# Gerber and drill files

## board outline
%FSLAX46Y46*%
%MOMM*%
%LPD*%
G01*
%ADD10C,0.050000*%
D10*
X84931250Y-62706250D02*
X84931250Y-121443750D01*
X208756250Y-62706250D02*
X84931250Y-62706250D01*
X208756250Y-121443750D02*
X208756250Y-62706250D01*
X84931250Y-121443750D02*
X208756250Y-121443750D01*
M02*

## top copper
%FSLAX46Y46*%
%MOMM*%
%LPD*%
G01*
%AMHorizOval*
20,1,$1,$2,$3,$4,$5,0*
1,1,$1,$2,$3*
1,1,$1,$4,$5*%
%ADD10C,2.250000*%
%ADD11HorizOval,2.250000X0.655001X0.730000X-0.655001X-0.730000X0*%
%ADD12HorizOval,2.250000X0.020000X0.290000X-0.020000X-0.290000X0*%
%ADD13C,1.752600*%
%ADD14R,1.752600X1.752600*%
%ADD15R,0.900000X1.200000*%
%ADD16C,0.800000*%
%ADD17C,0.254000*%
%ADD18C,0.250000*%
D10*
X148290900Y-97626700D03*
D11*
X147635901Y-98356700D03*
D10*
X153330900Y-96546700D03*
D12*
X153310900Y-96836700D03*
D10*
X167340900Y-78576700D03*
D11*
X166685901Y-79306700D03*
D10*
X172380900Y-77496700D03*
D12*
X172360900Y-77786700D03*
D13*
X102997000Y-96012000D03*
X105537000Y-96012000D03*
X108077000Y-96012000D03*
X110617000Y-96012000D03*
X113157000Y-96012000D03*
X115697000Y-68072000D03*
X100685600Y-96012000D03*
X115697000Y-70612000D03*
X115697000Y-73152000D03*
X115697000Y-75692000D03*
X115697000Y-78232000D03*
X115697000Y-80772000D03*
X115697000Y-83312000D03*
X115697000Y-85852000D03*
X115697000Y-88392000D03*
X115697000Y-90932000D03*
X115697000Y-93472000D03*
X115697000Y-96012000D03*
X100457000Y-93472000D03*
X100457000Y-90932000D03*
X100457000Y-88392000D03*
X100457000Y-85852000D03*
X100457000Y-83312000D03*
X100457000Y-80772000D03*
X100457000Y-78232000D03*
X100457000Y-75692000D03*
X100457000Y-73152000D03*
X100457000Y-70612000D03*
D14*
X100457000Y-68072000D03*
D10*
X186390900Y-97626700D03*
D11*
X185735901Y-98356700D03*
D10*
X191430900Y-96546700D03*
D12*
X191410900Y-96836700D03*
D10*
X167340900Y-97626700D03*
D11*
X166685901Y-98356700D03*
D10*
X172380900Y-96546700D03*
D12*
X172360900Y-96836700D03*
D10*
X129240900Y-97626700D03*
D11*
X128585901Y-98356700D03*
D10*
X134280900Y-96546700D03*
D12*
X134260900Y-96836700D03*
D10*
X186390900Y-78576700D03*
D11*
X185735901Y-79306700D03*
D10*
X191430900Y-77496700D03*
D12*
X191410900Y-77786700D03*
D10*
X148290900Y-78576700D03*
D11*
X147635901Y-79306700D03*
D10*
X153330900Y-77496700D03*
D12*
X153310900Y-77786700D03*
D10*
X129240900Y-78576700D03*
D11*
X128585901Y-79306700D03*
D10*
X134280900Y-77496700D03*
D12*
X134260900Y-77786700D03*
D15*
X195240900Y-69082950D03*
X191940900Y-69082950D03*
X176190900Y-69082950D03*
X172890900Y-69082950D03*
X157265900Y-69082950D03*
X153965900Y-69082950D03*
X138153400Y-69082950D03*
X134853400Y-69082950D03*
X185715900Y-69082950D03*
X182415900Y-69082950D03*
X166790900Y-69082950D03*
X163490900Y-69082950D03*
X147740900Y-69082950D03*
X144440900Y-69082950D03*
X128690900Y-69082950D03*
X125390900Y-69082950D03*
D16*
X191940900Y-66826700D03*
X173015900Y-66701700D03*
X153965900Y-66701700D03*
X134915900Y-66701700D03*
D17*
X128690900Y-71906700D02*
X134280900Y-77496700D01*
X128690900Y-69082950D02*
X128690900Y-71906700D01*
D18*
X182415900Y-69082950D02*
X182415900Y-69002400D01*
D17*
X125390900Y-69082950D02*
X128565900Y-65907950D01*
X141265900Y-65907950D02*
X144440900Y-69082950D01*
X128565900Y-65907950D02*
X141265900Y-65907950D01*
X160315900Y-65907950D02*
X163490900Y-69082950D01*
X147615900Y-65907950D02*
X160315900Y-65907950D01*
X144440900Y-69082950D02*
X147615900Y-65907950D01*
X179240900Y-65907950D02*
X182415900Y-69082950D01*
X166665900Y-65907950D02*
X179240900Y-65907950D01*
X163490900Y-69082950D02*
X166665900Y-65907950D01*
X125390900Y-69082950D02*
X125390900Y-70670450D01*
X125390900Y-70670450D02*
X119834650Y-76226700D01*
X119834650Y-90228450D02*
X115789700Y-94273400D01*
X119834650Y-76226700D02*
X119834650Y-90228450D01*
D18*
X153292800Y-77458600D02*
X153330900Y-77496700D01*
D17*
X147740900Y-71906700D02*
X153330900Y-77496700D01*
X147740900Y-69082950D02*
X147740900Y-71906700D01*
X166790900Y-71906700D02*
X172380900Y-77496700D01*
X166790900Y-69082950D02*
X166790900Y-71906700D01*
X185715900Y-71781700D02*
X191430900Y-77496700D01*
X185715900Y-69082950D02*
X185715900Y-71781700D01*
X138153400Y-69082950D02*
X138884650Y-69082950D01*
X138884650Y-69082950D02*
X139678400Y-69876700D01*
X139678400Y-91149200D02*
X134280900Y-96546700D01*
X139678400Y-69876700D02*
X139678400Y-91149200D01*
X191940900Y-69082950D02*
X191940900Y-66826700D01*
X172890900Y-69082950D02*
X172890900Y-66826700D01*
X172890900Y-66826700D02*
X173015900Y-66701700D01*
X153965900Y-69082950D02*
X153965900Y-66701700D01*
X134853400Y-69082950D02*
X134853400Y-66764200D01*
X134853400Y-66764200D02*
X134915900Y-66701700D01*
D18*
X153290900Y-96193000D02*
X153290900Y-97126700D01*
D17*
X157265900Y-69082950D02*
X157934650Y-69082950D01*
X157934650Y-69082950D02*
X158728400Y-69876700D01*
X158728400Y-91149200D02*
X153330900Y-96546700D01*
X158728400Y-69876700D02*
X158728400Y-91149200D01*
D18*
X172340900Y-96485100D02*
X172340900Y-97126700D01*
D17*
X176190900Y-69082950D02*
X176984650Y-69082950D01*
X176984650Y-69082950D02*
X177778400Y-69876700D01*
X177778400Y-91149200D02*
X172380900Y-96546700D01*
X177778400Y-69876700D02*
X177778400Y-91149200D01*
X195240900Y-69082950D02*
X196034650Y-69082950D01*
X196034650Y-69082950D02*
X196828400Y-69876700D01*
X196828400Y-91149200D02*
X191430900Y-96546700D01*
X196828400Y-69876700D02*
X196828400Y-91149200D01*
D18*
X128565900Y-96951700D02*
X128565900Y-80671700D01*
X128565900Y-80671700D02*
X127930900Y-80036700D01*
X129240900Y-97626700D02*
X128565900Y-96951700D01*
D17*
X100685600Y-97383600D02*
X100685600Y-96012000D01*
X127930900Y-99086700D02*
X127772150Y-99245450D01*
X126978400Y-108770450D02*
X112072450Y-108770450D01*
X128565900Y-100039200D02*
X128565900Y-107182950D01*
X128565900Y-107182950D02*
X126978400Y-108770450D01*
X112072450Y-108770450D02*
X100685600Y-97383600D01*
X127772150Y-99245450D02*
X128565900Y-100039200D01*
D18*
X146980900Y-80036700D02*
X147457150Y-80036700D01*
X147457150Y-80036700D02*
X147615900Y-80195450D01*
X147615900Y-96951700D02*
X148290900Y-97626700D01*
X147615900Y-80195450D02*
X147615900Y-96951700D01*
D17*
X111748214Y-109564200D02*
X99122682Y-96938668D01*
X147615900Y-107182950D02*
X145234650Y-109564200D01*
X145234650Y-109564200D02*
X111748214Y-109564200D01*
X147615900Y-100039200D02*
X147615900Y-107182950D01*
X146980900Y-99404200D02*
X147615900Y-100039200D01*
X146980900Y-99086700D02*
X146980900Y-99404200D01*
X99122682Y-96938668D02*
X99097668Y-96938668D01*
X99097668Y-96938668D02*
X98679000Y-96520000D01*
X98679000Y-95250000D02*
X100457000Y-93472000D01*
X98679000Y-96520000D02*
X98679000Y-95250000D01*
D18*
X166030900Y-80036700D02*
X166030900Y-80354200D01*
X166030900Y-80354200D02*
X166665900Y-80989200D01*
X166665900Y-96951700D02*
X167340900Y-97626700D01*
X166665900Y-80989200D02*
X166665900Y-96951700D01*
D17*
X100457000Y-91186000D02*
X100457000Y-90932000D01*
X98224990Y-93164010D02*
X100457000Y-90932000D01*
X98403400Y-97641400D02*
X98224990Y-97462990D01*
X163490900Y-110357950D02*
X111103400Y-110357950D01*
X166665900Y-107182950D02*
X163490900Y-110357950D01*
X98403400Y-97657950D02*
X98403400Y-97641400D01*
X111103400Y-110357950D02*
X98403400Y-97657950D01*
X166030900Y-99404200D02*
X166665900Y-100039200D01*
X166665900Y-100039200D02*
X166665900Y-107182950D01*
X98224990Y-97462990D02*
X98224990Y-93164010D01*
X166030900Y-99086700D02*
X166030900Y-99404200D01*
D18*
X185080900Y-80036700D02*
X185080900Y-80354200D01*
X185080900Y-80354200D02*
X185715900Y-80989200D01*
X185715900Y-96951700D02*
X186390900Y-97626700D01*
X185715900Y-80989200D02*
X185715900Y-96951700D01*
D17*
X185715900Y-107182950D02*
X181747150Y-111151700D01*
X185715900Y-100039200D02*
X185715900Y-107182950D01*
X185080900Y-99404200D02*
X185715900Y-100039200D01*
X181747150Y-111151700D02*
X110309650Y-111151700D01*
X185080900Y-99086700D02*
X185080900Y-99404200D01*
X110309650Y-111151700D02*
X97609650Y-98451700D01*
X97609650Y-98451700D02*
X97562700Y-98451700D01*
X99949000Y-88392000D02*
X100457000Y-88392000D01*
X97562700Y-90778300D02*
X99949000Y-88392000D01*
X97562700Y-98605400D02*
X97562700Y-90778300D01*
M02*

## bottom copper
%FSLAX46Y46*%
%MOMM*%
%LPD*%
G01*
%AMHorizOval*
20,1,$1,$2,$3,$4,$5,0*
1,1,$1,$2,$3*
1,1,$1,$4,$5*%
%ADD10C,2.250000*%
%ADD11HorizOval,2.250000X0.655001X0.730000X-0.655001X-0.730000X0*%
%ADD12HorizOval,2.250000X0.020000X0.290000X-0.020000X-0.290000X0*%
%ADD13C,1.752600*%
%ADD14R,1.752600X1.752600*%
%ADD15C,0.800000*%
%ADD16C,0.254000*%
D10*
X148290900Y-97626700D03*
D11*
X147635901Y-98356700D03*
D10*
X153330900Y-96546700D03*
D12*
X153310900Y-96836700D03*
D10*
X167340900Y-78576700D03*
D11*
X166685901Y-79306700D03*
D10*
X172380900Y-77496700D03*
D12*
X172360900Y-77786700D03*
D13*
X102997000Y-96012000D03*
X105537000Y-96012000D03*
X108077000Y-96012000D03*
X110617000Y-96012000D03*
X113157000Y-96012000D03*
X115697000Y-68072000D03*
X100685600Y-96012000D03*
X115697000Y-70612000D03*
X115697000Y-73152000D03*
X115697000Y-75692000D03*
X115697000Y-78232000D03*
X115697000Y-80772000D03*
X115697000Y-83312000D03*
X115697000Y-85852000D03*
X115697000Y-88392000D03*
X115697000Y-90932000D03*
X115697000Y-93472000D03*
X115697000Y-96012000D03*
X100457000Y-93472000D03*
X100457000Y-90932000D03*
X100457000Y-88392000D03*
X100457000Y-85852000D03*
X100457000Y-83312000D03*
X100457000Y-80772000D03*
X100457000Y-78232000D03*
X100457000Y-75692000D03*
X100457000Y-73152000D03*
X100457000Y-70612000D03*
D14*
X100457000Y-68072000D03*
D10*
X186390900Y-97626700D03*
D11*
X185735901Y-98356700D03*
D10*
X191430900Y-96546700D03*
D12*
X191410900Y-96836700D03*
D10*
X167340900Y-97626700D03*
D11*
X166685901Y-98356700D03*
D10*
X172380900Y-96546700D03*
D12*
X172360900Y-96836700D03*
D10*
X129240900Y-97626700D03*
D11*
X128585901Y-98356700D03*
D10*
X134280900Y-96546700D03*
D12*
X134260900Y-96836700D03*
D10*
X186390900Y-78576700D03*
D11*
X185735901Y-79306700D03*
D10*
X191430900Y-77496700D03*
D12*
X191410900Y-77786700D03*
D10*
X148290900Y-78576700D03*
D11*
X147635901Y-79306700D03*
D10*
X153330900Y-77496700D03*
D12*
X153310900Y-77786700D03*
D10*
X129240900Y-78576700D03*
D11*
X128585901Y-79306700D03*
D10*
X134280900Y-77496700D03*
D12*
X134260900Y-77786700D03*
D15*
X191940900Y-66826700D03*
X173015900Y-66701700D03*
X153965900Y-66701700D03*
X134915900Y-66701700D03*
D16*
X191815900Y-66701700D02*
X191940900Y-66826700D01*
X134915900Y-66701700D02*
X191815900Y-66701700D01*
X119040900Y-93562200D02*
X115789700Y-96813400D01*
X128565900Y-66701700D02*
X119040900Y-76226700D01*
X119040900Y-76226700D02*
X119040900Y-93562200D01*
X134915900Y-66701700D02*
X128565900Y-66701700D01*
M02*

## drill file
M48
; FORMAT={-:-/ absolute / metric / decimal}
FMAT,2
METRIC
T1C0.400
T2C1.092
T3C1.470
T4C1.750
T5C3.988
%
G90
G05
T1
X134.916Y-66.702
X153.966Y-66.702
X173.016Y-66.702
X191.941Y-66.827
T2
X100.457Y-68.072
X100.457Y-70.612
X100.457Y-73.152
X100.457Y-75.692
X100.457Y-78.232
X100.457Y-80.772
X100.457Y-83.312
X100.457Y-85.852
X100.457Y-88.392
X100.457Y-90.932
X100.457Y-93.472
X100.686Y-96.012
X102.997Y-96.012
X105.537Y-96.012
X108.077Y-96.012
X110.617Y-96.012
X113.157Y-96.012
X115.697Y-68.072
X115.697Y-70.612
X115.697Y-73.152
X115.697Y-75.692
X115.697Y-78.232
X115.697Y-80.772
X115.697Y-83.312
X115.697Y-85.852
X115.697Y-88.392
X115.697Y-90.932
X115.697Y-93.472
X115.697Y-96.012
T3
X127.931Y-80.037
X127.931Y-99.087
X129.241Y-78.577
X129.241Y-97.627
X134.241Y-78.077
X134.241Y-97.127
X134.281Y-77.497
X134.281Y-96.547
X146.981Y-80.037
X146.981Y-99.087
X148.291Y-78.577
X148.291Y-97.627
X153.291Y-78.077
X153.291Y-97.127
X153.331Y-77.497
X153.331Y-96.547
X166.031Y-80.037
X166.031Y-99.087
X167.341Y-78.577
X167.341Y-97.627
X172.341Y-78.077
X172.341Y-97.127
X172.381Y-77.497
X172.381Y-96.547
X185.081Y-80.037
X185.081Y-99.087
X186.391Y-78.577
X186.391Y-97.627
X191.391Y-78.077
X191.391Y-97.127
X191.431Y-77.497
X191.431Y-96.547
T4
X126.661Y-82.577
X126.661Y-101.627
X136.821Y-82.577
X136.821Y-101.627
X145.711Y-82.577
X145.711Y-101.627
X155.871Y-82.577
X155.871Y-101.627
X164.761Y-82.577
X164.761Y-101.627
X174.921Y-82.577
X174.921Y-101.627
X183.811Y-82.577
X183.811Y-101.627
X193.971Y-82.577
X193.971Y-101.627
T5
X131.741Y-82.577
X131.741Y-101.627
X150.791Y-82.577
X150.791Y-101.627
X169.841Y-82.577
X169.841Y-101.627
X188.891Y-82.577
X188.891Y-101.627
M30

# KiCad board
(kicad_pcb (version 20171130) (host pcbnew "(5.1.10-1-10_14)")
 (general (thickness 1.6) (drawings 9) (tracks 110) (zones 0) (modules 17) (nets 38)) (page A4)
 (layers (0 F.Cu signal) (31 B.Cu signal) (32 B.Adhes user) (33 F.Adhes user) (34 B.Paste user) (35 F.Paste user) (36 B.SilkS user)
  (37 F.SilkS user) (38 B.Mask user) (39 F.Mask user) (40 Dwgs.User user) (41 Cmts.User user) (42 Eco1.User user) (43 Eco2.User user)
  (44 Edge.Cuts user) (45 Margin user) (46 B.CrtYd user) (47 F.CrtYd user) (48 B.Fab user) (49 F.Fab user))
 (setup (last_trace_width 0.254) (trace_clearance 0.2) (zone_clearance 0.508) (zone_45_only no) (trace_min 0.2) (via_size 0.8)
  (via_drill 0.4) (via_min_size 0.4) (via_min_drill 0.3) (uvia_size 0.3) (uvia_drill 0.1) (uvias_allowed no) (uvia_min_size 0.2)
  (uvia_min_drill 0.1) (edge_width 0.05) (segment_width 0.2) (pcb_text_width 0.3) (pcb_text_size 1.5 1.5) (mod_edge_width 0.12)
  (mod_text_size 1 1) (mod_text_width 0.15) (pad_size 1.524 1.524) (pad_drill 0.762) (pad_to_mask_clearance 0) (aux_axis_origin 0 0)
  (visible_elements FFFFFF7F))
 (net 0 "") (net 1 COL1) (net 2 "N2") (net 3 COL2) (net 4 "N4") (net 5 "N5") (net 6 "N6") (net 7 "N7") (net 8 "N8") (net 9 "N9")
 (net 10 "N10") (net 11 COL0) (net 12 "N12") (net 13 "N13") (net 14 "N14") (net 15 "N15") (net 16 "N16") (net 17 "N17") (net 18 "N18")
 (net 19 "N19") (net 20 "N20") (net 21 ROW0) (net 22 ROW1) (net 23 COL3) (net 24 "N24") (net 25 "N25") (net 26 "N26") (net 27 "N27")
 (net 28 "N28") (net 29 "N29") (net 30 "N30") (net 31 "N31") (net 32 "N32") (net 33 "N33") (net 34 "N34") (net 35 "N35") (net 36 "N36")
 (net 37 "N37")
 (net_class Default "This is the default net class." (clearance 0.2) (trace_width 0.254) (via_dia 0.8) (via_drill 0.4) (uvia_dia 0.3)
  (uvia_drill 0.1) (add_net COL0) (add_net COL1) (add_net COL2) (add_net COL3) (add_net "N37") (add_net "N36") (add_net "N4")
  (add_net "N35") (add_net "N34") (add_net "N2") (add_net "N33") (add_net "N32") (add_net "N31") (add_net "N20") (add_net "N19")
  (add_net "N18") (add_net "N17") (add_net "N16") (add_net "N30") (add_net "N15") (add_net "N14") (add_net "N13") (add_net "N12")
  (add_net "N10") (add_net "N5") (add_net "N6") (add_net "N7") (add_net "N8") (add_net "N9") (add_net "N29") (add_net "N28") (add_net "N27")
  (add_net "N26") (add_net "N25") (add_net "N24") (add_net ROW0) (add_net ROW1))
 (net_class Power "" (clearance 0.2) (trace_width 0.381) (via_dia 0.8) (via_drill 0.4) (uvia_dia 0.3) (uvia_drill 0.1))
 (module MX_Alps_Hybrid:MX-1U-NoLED (layer F.Cu) (at 150.7909 101.6267)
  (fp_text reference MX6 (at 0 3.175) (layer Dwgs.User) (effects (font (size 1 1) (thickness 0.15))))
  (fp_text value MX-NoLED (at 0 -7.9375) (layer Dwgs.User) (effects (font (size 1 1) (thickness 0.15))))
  (pad "" np_thru_hole circle (at 5.08 0 48.0996) (size 1.75 1.75) (drill 1.75) (layers *.Cu *.Mask))
  (pad "" np_thru_hole circle (at -5.08 0 48.0996) (size 1.75 1.75) (drill 1.75) (layers *.Cu *.Mask))
  (pad 1 thru_hole circle (at -2.5 -4) (size 2.25 2.25) (drill 1.47) (layers *.Cu B.Mask) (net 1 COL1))
  (pad "" np_thru_hole circle (at 0 0) (size 3.9878 3.9878) (drill 3.9878) (layers *.Cu *.Mask))
  (pad 1 thru_hole oval (at -3.81 -2.54 48.0996) (size 4.211556 2.25) (drill 1.47 (offset 0.980778 0)) (layers *.Cu B.Mask) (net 1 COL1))
  (pad 2 thru_hole circle (at 2.54 -5.08) (size 2.25 2.25) (drill 1.47) (layers *.Cu B.Mask) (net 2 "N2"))
  (pad 2 thru_hole oval (at 2.5 -4.5 86.0548) (size 2.831378 2.25) (drill 1.47 (offset 0.290689 0)) (layers *.Cu B.Mask) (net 2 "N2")))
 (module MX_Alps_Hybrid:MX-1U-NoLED (layer F.Cu) (at 169.8409 82.5767)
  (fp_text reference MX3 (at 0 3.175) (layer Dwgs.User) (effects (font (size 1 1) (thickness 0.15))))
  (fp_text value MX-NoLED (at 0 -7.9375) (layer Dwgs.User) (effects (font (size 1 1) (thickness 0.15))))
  (pad "" np_thru_hole circle (at 5.08 0 48.0996) (size 1.75 1.75) (drill 1.75) (layers *.Cu *.Mask))
  (pad "" np_thru_hole circle (at -5.08 0 48.0996) (size 1.75 1.75) (drill 1.75) (layers *.Cu *.Mask))
  (pad 1 thru_hole circle (at -2.5 -4) (size 2.25 2.25) (drill 1.47) (layers *.Cu B.Mask) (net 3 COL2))
  (pad "" np_thru_hole circle (at 0 0) (size 3.9878 3.9878) (drill 3.9878) (layers *.Cu *.Mask))
  (pad 1 thru_hole oval (at -3.81 -2.54 48.0996) (size 4.211556 2.25) (drill 1.47 (offset 0.980778 0)) (layers *.Cu B.Mask) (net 3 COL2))
  (pad 2 thru_hole circle (at 2.54 -5.08) (size 2.25 2.25) (drill 1.47) (layers *.Cu B.Mask) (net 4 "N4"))
  (pad 2 thru_hole oval (at 2.5 -4.5 86.0548) (size 2.831378 2.25) (drill 1.47 (offset 0.290689 0)) (layers *.Cu B.Mask) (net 4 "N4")))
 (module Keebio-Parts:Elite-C (layer F.Cu) (at 108.077 82.042 270)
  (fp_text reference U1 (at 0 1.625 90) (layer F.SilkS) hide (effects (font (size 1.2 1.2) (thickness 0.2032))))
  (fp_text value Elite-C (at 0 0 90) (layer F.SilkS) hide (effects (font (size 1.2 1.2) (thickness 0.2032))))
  (pad 25 thru_hole circle (at 13.97 5.08 270) (size 1.7526 1.7526) (drill 1.0922) (layers *.Cu *.SilkS *.Mask) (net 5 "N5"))
  (pad 26 thru_hole circle (at 13.97 2.54 270) (size 1.7526 1.7526) (drill 1.0922) (layers *.Cu *.SilkS *.Mask) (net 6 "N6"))
  (pad 27 thru_hole circle (at 13.97 0 270) (size 1.7526 1.7526) (drill 1.0922) (layers *.Cu *.SilkS *.Mask) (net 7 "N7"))
  (pad 28 thru_hole circle (at 13.97 -2.54 270) (size 1.7526 1.7526) (drill 1.0922) (layers *.Cu *.SilkS *.Mask) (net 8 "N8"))
  (pad 29 thru_hole circle (at 13.97 -5.08 270) (size 1.7526 1.7526) (drill 1.0922) (layers *.Cu *.SilkS *.Mask) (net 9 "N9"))
  (pad 24 thru_hole circle (at -13.97 -7.62 270) (size 1.7526 1.7526) (drill 1.0922) (layers *.Cu *.SilkS *.Mask) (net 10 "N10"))
  (pad 12 thru_hole circle (at 13.97 7.3914 270) (size 1.7526 1.7526) (drill 1.0922) (layers *.Cu *.SilkS *.Mask) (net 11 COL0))
  (pad 23 thru_hole circle (at -11.43 -7.62 270) (size 1.7526 1.7526) (drill 1.0922) (layers *.Cu *.SilkS *.Mask) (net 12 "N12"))
  (pad 22 thru_hole circle (at -8.89 -7.62 270) (size 1.7526 1.7526) (drill 1.0922) (layers *.Cu *.SilkS *.Mask) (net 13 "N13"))
  (pad 21 thru_hole circle (at -6.35 -7.62 270) (size 1.7526 1.7526) (drill 1.0922) (layers *.Cu *.SilkS *.Mask) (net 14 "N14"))
  (pad 20 thru_hole circle (at -3.81 -7.62 270) (size 1.7526 1.7526) (drill 1.0922) (layers *.Cu *.SilkS *.Mask) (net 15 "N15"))
  (pad 19 thru_hole circle (at -1.27 -7.62 270) (size 1.7526 1.7526) (drill 1.0922) (layers *.Cu *.SilkS *.Mask) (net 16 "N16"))
  (pad 18 thru_hole circle (at 1.27 -7.62 270) (size 1.7526 1.7526) (drill 1.0922) (layers *.Cu *.SilkS *.Mask) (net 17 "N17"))
  (pad 17 thru_hole circle (at 3.81 -7.62 270) (size 1.7526 1.7526) (drill 1.0922) (layers *.Cu *.SilkS *.Mask) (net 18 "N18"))
  (pad 16 thru_hole circle (at 6.35 -7.62 270) (size 1.7526 1.7526) (drill 1.0922) (layers *.Cu *.SilkS *.Mask) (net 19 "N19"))
  (pad 15 thru_hole circle (at 8.89 -7.62 270) (size 1.7526 1.7526) (drill 1.0922) (layers *.Cu *.SilkS *.Mask) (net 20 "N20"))
  (pad 14 thru_hole circle (at 11.43 -7.62 270) (size 1.7526 1.7526) (drill 1.0922) (layers *.Cu *.SilkS *.Mask) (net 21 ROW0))
  (pad 13 thru_hole circle (at 13.97 -7.62 270) (size 1.7526 1.7526) (drill 1.0922) (layers *.Cu *.SilkS *.Mask) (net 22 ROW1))
  (pad 11 thru_hole circle (at 11.43 7.62 270) (size 1.7526 1.7526) (drill 1.0922) (layers *.Cu *.SilkS *.Mask) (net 1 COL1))
  (pad 10 thru_hole circle (at 8.89 7.62 270) (size 1.7526 1.7526) (drill 1.0922) (layers *.Cu *.SilkS *.Mask) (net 3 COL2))
  (pad 9 thru_hole circle (at 6.35 7.62 270) (size 1.7526 1.7526) (drill 1.0922) (layers *.Cu *.SilkS *.Mask) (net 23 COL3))
  (pad 8 thru_hole circle (at 3.81 7.62 270) (size 1.7526 1.7526) (drill 1.0922) (layers *.Cu *.SilkS *.Mask) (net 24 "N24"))
  (pad 7 thru_hole circle (at 1.27 7.62 270) (size 1.7526 1.7526) (drill 1.0922) (layers *.Cu *.SilkS *.Mask) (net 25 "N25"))
  (pad 6 thru_hole circle (at -1.27 7.62 270) (size 1.7526 1.7526) (drill 1.0922) (layers *.Cu *.SilkS *.Mask) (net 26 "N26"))
  (pad 5 thru_hole circle (at -3.81 7.62 270) (size 1.7526 1.7526) (drill 1.0922) (layers *.Cu *.SilkS *.Mask) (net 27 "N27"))
  (pad 4 thru_hole circle (at -6.35 7.62 270) (size 1.7526 1.7526) (drill 1.0922) (layers *.Cu *.SilkS *.Mask) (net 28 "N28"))
  (pad 3 thru_hole circle (at -8.89 7.62 270) (size 1.7526 1.7526) (drill 1.0922) (layers *.Cu *.SilkS *.Mask) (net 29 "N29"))
  (pad 2 thru_hole circle (at -11.43 7.62 270) (size 1.7526 1.7526) (drill 1.0922) (layers *.Cu *.SilkS *.Mask) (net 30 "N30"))
  (pad 1 thru_hole rect (at -13.97 7.62 270) (size 1.7526 1.7526) (drill 1.0922) (layers *.Cu *.SilkS *.Mask) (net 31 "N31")))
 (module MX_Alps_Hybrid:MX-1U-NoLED (layer F.Cu) (at 188.8909 101.6267)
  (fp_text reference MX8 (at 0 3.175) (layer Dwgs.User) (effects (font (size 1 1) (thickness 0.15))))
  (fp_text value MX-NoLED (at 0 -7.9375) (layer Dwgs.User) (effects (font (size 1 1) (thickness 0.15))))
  (pad "" np_thru_hole circle (at 5.08 0 48.0996) (size 1.75 1.75) (drill 1.75) (layers *.Cu *.Mask))
  (pad "" np_thru_hole circle (at -5.08 0 48.0996) (size 1.75 1.75) (drill 1.75) (layers *.Cu *.Mask))
  (pad 1 thru_hole circle (at -2.5 -4) (size 2.25 2.25) (drill 1.47) (layers *.Cu B.Mask) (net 23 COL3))
  (pad "" np_thru_hole circle (at 0 0) (size 3.9878 3.9878) (drill 3.9878) (layers *.Cu *.Mask))
  (pad 1 thru_hole oval (at -3.81 -2.54 48.0996) (size 4.211556 2.25) (drill 1.47 (offset 0.980778 0)) (layers *.Cu B.Mask) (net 23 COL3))
  (pad 2 thru_hole circle (at 2.54 -5.08) (size 2.25 2.25) (drill 1.47) (layers *.Cu B.Mask) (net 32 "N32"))
  (pad 2 thru_hole oval (at 2.5 -4.5 86.0548) (size 2.831378 2.25) (drill 1.47 (offset 0.290689 0)) (layers *.Cu B.Mask) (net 32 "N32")))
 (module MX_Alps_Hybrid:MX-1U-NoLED (layer F.Cu) (at 169.8409 101.6267)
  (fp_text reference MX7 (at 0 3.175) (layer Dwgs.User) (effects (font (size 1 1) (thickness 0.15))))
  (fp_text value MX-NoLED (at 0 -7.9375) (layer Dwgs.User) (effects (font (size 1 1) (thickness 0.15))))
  (pad "" np_thru_hole circle (at 5.08 0 48.0996) (size 1.75 1.75) (drill 1.75) (layers *.Cu *.Mask))
  (pad "" np_thru_hole circle (at -5.08 0 48.0996) (size 1.75 1.75) (drill 1.75) (layers *.Cu *.Mask))
  (pad 1 thru_hole circle (at -2.5 -4) (size 2.25 2.25) (drill 1.47) (layers *.Cu B.Mask) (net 3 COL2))
  (pad "" np_thru_hole circle (at 0 0) (size 3.9878 3.9878) (drill 3.9878) (layers *.Cu *.Mask))
  (pad 1 thru_hole oval (at -3.81 -2.54 48.0996) (size 4.211556 2.25) (drill 1.47 (offset 0.980778 0)) (layers *.Cu B.Mask) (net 3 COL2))
  (pad 2 thru_hole circle (at 2.54 -5.08) (size 2.25 2.25) (drill 1.47) (layers *.Cu B.Mask) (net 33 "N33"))
  (pad 2 thru_hole oval (at 2.5 -4.5 86.0548) (size 2.831378 2.25) (drill 1.47 (offset 0.290689 0)) (layers *.Cu B.Mask) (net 33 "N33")))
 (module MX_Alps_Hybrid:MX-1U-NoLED (layer F.Cu) (at 131.7409 101.6267)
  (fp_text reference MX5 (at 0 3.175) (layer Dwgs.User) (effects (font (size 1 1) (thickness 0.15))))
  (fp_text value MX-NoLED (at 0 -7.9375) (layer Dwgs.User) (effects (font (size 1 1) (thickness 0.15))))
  (pad "" np_thru_hole circle (at 5.08 0 48.0996) (size 1.75 1.75) (drill 1.75) (layers *.Cu *.Mask))
  (pad "" np_thru_hole circle (at -5.08 0 48.0996) (size 1.75 1.75) (drill 1.75) (layers *.Cu *.Mask))
  (pad 1 thru_hole circle (at -2.5 -4) (size 2.25 2.25) (drill 1.47) (layers *.Cu B.Mask) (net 11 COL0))
  (pad "" np_thru_hole circle (at 0 0) (size 3.9878 3.9878) (drill 3.9878) (layers *.Cu *.Mask))
  (pad 1 thru_hole oval (at -3.81 -2.54 48.0996) (size 4.211556 2.25) (drill 1.47 (offset 0.980778 0)) (layers *.Cu B.Mask) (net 11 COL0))
  (pad 2 thru_hole circle (at 2.54 -5.08) (size 2.25 2.25) (drill 1.47) (layers *.Cu B.Mask) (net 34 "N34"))
  (pad 2 thru_hole oval (at 2.5 -4.5 86.0548) (size 2.831378 2.25) (drill 1.47 (offset 0.290689 0)) (layers *.Cu B.Mask) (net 34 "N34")))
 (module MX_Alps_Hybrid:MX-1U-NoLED (layer F.Cu) (at 188.8909 82.5767)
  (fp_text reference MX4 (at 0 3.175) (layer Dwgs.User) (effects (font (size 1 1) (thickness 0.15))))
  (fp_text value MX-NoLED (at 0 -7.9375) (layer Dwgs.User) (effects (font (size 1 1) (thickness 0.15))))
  (pad "" np_thru_hole circle (at 5.08 0 48.0996) (size 1.75 1.75) (drill 1.75) (layers *.Cu *.Mask))
  (pad "" np_thru_hole circle (at -5.08 0 48.0996) (size 1.75 1.75) (drill 1.75) (layers *.Cu *.Mask))
  (pad 1 thru_hole circle (at -2.5 -4) (size 2.25 2.25) (drill 1.47) (layers *.Cu B.Mask) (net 23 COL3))
  (pad "" np_thru_hole circle (at 0 0) (size 3.9878 3.9878) (drill 3.9878) (layers *.Cu *.Mask))
  (pad 1 thru_hole oval (at -3.81 -2.54 48.0996) (size 4.211556 2.25) (drill 1.47 (offset 0.980778 0)) (layers *.Cu B.Mask) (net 23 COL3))
  (pad 2 thru_hole circle (at 2.54 -5.08) (size 2.25 2.25) (drill 1.47) (layers *.Cu B.Mask) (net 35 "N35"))
  (pad 2 thru_hole oval (at 2.5 -4.5 86.0548) (size 2.831378 2.25) (drill 1.47 (offset 0.290689 0)) (layers *.Cu B.Mask) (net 35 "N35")))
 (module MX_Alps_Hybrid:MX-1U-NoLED (layer F.Cu) (at 150.7909 82.5767)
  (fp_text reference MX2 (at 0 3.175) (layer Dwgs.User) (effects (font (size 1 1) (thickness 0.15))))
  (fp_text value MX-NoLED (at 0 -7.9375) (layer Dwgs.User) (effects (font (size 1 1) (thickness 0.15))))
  (pad "" np_thru_hole circle (at 5.08 0 48.0996) (size 1.75 1.75) (drill 1.75) (layers *.Cu *.Mask))
  (pad "" np_thru_hole circle (at -5.08 0 48.0996) (size 1.75 1.75) (drill 1.75) (layers *.Cu *.Mask))
  (pad 1 thru_hole circle (at -2.5 -4) (size 2.25 2.25) (drill 1.47) (layers *.Cu B.Mask) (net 1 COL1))
  (pad "" np_thru_hole circle (at 0 0) (size 3.9878 3.9878) (drill 3.9878) (layers *.Cu *.Mask))
  (pad 1 thru_hole oval (at -3.81 -2.54 48.0996) (size 4.211556 2.25) (drill 1.47 (offset 0.980778 0)) (layers *.Cu B.Mask) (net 1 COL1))
  (pad 2 thru_hole circle (at 2.54 -5.08) (size 2.25 2.25) (drill 1.47) (layers *.Cu B.Mask) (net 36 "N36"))
  (pad 2 thru_hole oval (at 2.5 -4.5 86.0548) (size 2.831378 2.25) (drill 1.47 (offset 0.290689 0)) (layers *.Cu B.Mask) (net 36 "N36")))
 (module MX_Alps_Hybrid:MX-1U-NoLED (layer F.Cu) (at 131.7409 82.5767)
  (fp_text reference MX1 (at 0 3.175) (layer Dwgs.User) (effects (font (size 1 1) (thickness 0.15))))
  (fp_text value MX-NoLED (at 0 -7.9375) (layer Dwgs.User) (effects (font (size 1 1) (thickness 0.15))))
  (pad "" np_thru_hole circle (at 5.08 0 48.0996) (size 1.75 1.75) (drill 1.75) (layers *.Cu *.Mask))
  (pad "" np_thru_hole circle (at -5.08 0 48.0996) (size 1.75 1.75) (drill 1.75) (layers *.Cu *.Mask))
  (pad 1 thru_hole circle (at -2.5 -4) (size 2.25 2.25) (drill 1.47) (layers *.Cu B.Mask) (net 11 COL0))
  (pad "" np_thru_hole circle (at 0 0) (size 3.9878 3.9878) (drill 3.9878) (layers *.Cu *.Mask))
  (pad 1 thru_hole oval (at -3.81 -2.54 48.0996) (size 4.211556 2.25) (drill 1.47 (offset 0.980778 0)) (layers *.Cu B.Mask) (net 11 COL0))
  (pad 2 thru_hole circle (at 2.54 -5.08) (size 2.25 2.25) (drill 1.47) (layers *.Cu B.Mask) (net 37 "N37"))
  (pad 2 thru_hole oval (at 2.5 -4.5 86.0548) (size 2.831378 2.25) (drill 1.47 (offset 0.290689 0)) (layers *.Cu B.Mask) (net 37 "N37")))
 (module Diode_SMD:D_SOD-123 (layer F.Cu) (at 193.5909 69.08295)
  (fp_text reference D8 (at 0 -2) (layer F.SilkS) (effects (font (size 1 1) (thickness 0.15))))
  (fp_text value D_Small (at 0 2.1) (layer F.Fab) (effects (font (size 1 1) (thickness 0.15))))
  (pad 2 smd rect (at 1.65 0) (size 0.9 1.2) (layers F.Cu F.Paste F.Mask) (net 32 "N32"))
  (pad 1 smd rect (at -1.65 0) (size 0.9 1.2) (layers F.Cu F.Paste F.Mask) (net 22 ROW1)))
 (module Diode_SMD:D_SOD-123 (layer F.Cu) (at 174.5409 69.08295)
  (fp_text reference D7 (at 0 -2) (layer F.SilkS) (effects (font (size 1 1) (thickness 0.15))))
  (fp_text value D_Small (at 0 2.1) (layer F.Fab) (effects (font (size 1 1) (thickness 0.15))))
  (pad 2 smd rect (at 1.65 0) (size 0.9 1.2) (layers F.Cu F.Paste F.Mask) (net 33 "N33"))
  (pad 1 smd rect (at -1.65 0) (size 0.9 1.2) (layers F.Cu F.Paste F.Mask) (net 22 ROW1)))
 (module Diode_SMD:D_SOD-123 (layer F.Cu) (at 155.6159 69.08295)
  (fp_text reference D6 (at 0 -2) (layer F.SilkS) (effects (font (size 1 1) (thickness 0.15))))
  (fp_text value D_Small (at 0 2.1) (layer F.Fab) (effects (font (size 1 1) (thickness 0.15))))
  (pad 2 smd rect (at 1.65 0) (size 0.9 1.2) (layers F.Cu F.Paste F.Mask) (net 2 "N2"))
  (pad 1 smd rect (at -1.65 0) (size 0.9 1.2) (layers F.Cu F.Paste F.Mask) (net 22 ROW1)))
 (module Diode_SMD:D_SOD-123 (layer F.Cu) (at 136.5034 69.08295)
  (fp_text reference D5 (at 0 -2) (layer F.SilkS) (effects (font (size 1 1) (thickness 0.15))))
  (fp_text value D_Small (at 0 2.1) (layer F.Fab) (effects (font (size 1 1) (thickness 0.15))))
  (pad 2 smd rect (at 1.65 0) (size 0.9 1.2) (layers F.Cu F.Paste F.Mask) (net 34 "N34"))
  (pad 1 smd rect (at -1.65 0) (size 0.9 1.2) (layers F.Cu F.Paste F.Mask) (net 22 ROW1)))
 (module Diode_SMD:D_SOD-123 (layer F.Cu) (at 184.0659 69.08295)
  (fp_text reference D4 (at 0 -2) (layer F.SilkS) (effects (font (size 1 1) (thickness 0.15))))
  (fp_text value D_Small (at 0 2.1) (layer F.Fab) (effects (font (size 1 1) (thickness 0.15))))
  (pad 2 smd rect (at 1.65 0) (size 0.9 1.2) (layers F.Cu F.Paste F.Mask) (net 35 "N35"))
  (pad 1 smd rect (at -1.65 0) (size 0.9 1.2) (layers F.Cu F.Paste F.Mask) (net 21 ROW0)))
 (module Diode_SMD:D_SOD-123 (layer F.Cu) (at 165.1409 69.08295)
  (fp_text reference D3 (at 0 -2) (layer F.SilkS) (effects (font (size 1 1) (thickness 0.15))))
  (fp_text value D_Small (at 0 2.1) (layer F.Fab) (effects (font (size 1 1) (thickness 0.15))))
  (pad 2 smd rect (at 1.65 0) (size 0.9 1.2) (layers F.Cu F.Paste F.Mask) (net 4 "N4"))
  (pad 1 smd rect (at -1.65 0) (size 0.9 1.2) (layers F.Cu F.Paste F.Mask) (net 21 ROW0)))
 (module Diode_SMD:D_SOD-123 (layer F.Cu) (at 146.0909 69.08295)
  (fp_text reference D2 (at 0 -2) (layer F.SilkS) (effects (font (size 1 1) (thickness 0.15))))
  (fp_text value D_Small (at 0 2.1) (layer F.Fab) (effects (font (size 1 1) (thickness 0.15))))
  (pad 2 smd rect (at 1.65 0) (size 0.9 1.2) (layers F.Cu F.Paste F.Mask) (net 36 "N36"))
  (pad 1 smd rect (at -1.65 0) (size 0.9 1.2) (layers F.Cu F.Paste F.Mask) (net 21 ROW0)))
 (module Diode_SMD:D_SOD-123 (layer F.Cu) (at 127.0409 69.08295)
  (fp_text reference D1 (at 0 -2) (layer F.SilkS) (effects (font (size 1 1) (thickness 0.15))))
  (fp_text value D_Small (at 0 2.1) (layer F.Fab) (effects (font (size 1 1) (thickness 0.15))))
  (pad 2 smd rect (at 1.65 0) (size 0.9 1.2) (layers F.Cu F.Paste F.Mask) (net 37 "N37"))
  (pad 1 smd rect (at -1.65 0) (size 0.9 1.2) (layers F.Cu F.Paste F.Mask) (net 21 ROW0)))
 (gr_line (start 84.93125 62.70625) (end 84.93125 121.44375) (layer Edge.Cuts) (width 0.05))
 (gr_line (start 208.75625 62.70625) (end 84.93125 62.70625) (layer Edge.Cuts) (width 0.05))
 (gr_line (start 208.75625 121.44375) (end 208.75625 62.70625) (layer Edge.Cuts) (width 0.05))
 (gr_line (start 84.93125 121.44375) (end 208.75625 121.44375) (layer Edge.Cuts) (width 0.05))
 (segment (start 128.6909 71.9067) (end 134.2809 77.4967) (width 0.254) (layer F.Cu) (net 37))
 (segment (start 128.6909 69.08295) (end 128.6909 71.9067) (width 0.254) (layer F.Cu) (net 37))
 (segment (start 182.4159 69.08295) (end 182.4159 69.0024) (width 0.25) (layer F.Cu) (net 21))
 (segment (start 125.3909 69.08295) (end 128.5659 65.90795) (width 0.254) (layer F.Cu) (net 21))
 (segment (start 141.2659 65.90795) (end 144.4409 69.08295) (width 0.254) (layer F.Cu) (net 21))
 (segment (start 128.5659 65.90795) (end 141.2659 65.90795) (width 0.254) (layer F.Cu) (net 21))
 (segment (start 160.3159 65.90795) (end 163.4909 69.08295) (width 0.254) (layer F.Cu) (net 21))
 (segment (start 147.6159 65.90795) (end 160.3159 65.90795) (width 0.254) (layer F.Cu) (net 21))
 (segment (start 144.4409 69.08295) (end 147.6159 65.90795) (width 0.254) (layer F.Cu) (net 21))
 (segment (start 179.2409 65.90795) (end 182.4159 69.08295) (width 0.254) (layer F.Cu) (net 21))
 (segment (start 166.6659 65.90795) (end 179.2409 65.90795) (width 0.254) (layer F.Cu) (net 21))
 (segment (start 163.4909 69.08295) (end 166.6659 65.90795) (width 0.254) (layer F.Cu) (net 21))
 (segment (start 125.3909 69.08295) (end 125.3909 70.67045) (width 0.254) (layer F.Cu) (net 21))
 (segment (start 125.3909 70.67045) (end 119.83465 76.2267) (width 0.254) (layer F.Cu) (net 21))
 (segment (start 119.83465 90.22845) (end 115.7897 94.2734) (width 0.254) (layer F.Cu) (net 21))
 (segment (start 119.83465 76.2267) (end 119.83465 90.22845) (width 0.254) (layer F.Cu) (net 21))
 (segment (start 153.2928 77.4586) (end 153.3309 77.4967) (width 0.25) (layer F.Cu) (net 36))
 (segment (start 147.7409 71.9067) (end 153.3309 77.4967) (width 0.254) (layer F.Cu) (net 36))
 (segment (start 147.7409 69.08295) (end 147.7409 71.9067) (width 0.254) (layer F.Cu) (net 36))
 (segment (start 166.7909 71.9067) (end 172.3809 77.4967) (width 0.254) (layer F.Cu) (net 4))
 (segment (start 166.7909 69.08295) (end 166.7909 71.9067) (width 0.254) (layer F.Cu) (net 4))
 (segment (start 185.7159 71.7817) (end 191.4309 77.4967) (width 0.254) (layer F.Cu) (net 35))
 (segment (start 185.7159 69.08295) (end 185.7159 71.7817) (width 0.254) (layer F.Cu) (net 35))
 (segment (start 138.1534 69.08295) (end 138.88465 69.08295) (width 0.254) (layer F.Cu) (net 34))
 (segment (start 138.88465 69.08295) (end 139.6784 69.8767) (width 0.254) (layer F.Cu) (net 34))
 (segment (start 139.6784 91.1492) (end 134.2809 96.5467) (width 0.254) (layer F.Cu) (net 34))
 (segment (start 139.6784 69.8767) (end 139.6784 91.1492) (width 0.254) (layer F.Cu) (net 34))
 (segment (start 191.9409 69.08295) (end 191.9409 66.8267) (width 0.254) (layer F.Cu) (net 22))
 (via (at 191.9409 66.8267) (size 0.8) (drill 0.4) (layers F.Cu B.Cu) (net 22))
 (segment (start 172.8909 69.08295) (end 172.8909 66.8267) (width 0.254) (layer F.Cu) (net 22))
 (via (at 173.0159 66.7017) (size 0.8) (drill 0.4) (layers F.Cu B.Cu) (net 22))
 (segment (start 172.8909 66.8267) (end 173.0159 66.7017) (width 0.254) (layer F.Cu) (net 22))
 (segment (start 153.9659 69.08295) (end 153.9659 66.7017) (width 0.254) (layer F.Cu) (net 22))
 (via (at 153.9659 66.7017) (size 0.8) (drill 0.4) (layers F.Cu B.Cu) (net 22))
 (segment (start 134.8534 69.08295) (end 134.8534 66.7642) (width 0.254) (layer F.Cu) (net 22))
 (via (at 134.9159 66.7017) (size 0.8) (drill 0.4) (layers F.Cu B.Cu) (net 22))
 (segment (start 134.8534 66.7642) (end 134.9159 66.7017) (width 0.254) (layer F.Cu) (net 22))
 (segment (start 191.8159 66.7017) (end 191.9409 66.8267) (width 0.254) (layer B.Cu) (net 22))
 (segment (start 134.9159 66.7017) (end 191.8159 66.7017) (width 0.254) (layer B.Cu) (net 22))
 (segment (start 119.0409 93.5622) (end 115.7897 96.8134) (width 0.254) (layer B.Cu) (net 22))
 (segment (start 128.5659 66.7017) (end 119.0409 76.2267) (width 0.254) (layer B.Cu) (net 22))
 (segment (start 119.0409 76.2267) (end 119.0409 93.5622) (width 0.254) (layer B.Cu) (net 22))
 (segment (start 134.9159 66.7017) (end 128.5659 66.7017) (width 0.254) (layer B.Cu) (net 22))
 (segment (start 153.2909 96.193) (end 153.2909 97.1267) (width 0.25) (layer F.Cu) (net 2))
 (segment (start 157.2659 69.08295) (end 157.93465 69.08295) (width 0.254) (layer F.Cu) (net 2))
 (segment (start 157.93465 69.08295) (end 158.7284 69.8767) (width 0.254) (layer F.Cu) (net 2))
 (segment (start 158.7284 91.1492) (end 153.3309 96.5467) (width 0.254) (layer F.Cu) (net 2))
 (segment (start 158.7284 69.8767) (end 158.7284 91.1492) (width 0.254) (layer F.Cu) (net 2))
 (segment (start 172.3409 96.4851) (end 172.3409 97.1267) (width 0.25) (layer F.Cu) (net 33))
 (segment (start 176.1909 69.08295) (end 176.98465 69.08295) (width 0.254) (layer F.Cu) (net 33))
 (segment (start 176.98465 69.08295) (end 177.7784 69.8767) (width 0.254) (layer F.Cu) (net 33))
 (segment (start 177.7784 91.1492) (end 172.3809 96.5467) (width 0.254) (layer F.Cu) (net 33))
 (segment (start 177.7784 69.8767) (end 177.7784 91.1492) (width 0.254) (layer F.Cu) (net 33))
 (segment (start 195.2409 69.08295) (end 196.03465 69.08295) (width 0.254) (layer F.Cu) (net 32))
 (segment (start 196.03465 69.08295) (end 196.8284 69.8767) (width 0.254) (layer F.Cu) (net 32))
 (segment (start 196.8284 91.1492) (end 191.4309 96.5467) (width 0.254) (layer F.Cu) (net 32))
 (segment (start 196.8284 69.8767) (end 196.8284 91.1492) (width 0.254) (layer F.Cu) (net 32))
 (segment (start 128.5659 96.9517) (end 128.5659 80.6717) (width 0.25) (layer F.Cu) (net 11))
 (segment (start 128.5659 80.6717) (end 127.9309 80.0367) (width 0.25) (layer F.Cu) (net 11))
 (segment (start 129.2409 97.6267) (end 128.5659 96.9517) (width 0.25) (layer F.Cu) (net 11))
 (segment (start 100.6856 97.3836) (end 100.6856 96.012) (width 0.254) (layer F.Cu) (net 11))
 (segment (start 127.9309 99.0867) (end 127.77215 99.24545) (width 0.254) (layer F.Cu) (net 11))
 (segment (start 126.9784 108.77045) (end 112.07245 108.77045) (width 0.254) (layer F.Cu) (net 11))
 (segment (start 128.5659 100.0392) (end 128.5659 107.18295) (width 0.254) (layer F.Cu) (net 11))
 (segment (start 128.5659 107.18295) (end 126.9784 108.77045) (width 0.254) (layer F.Cu) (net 11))
 (segment (start 112.07245 108.77045) (end 100.6856 97.3836) (width 0.254) (layer F.Cu) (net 11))
 (segment (start 127.77215 99.24545) (end 128.5659 100.0392) (width 0.254) (layer F.Cu) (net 11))
 (segment (start 146.9809 80.0367) (end 147.45715 80.0367) (width 0.25) (layer F.Cu) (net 1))
 (segment (start 147.45715 80.0367) (end 147.6159 80.19545) (width 0.25) (layer F.Cu) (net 1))
 (segment (start 147.6159 96.9517) (end 148.2909 97.6267) (width 0.25) (layer F.Cu) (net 1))
 (segment (start 147.6159 80.19545) (end 147.6159 96.9517) (width 0.25) (layer F.Cu) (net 1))
 (segment (start 111.748214 109.5642) (end 99.122682 96.938668) (width 0.254) (layer F.Cu) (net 1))
 (segment (start 147.6159 107.18295) (end 145.23465 109.5642) (width 0.254) (layer F.Cu) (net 1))
 (segment (start 145.23465 109.5642) (end 111.748214 109.5642) (width 0.254) (layer F.Cu) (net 1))
 (segment (start 147.6159 100.0392) (end 147.6159 107.18295) (width 0.254) (layer F.Cu) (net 1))
 (segment (start 146.9809 99.4042) (end 147.6159 100.0392) (width 0.254) (layer F.Cu) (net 1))
 (segment (start 146.9809 99.0867) (end 146.9809 99.4042) (width 0.254) (layer F.Cu) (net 1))
 (segment (start 99.122682 96.938668) (end 99.097668 96.938668) (width 0.254) (layer F.Cu) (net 1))
 (segment (start 99.097668 96.938668) (end 98.679 96.52) (width 0.254) (layer F.Cu) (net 1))
 (segment (start 98.679 95.25) (end 100.457 93.472) (width 0.254) (layer F.Cu) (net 1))
 (segment (start 98.679 96.52) (end 98.679 95.25) (width 0.254) (layer F.Cu) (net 1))
 (segment (start 166.0309 80.0367) (end 166.0309 80.3542) (width 0.25) (layer F.Cu) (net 3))
 (segment (start 166.0309 80.3542) (end 166.6659 80.9892) (width 0.25) (layer F.Cu) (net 3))
 (segment (start 166.6659 96.9517) (end 167.3409 97.6267) (width 0.25) (layer F.Cu) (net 3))
 (segment (start 166.6659 80.9892) (end 166.6659 96.9517) (width 0.25) (layer F.Cu) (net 3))
 (segment (start 100.457 91.186) (end 100.457 90.932) (width 0.254) (layer F.Cu) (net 3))
 (segment (start 98.22499 93.16401) (end 100.457 90.932) (width 0.254) (layer F.Cu) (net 3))
 (segment (start 98.4034 97.6414) (end 98.22499 97.46299) (width 0.254) (layer F.Cu) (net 3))
 (segment (start 163.4909 110.35795) (end 111.1034 110.35795) (width 0.254) (layer F.Cu) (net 3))
 (segment (start 166.6659 107.18295) (end 163.4909 110.35795) (width 0.254) (layer F.Cu) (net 3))
 (segment (start 98.4034 97.65795) (end 98.4034 97.6414) (width 0.254) (layer F.Cu) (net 3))
 (segment (start 111.1034 110.35795) (end 98.4034 97.65795) (width 0.254) (layer F.Cu) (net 3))
 (segment (start 166.0309 99.4042) (end 166.6659 100.0392) (width 0.254) (layer F.Cu) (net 3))
 (segment (start 166.6659 100.0392) (end 166.6659 107.18295) (width 0.254) (layer F.Cu) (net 3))
 (segment (start 98.22499 97.46299) (end 98.22499 93.16401) (width 0.254) (layer F.Cu) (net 3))
 (segment (start 166.0309 99.0867) (end 166.0309 99.4042) (width 0.254) (layer F.Cu) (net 3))
 (segment (start 185.0809 80.0367) (end 185.0809 80.3542) (width 0.25) (layer F.Cu) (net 23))
 (segment (start 185.0809 80.3542) (end 185.7159 80.9892) (width 0.25) (layer F.Cu) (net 23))
 (segment (start 185.7159 96.9517) (end 186.3909 97.6267) (width 0.25) (layer F.Cu) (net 23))
 (segment (start 185.7159 80.9892) (end 185.7159 96.9517) (width 0.25) (layer F.Cu) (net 23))
 (segment (start 185.7159 107.18295) (end 181.74715 111.1517) (width 0.254) (layer F.Cu) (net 23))
 (segment (start 185.7159 100.0392) (end 185.7159 107.18295) (width 0.254) (layer F.Cu) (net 23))
 (segment (start 185.0809 99.4042) (end 185.7159 100.0392) (width 0.254) (layer F.Cu) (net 23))
 (segment (start 181.74715 111.1517) (end 110.30965 111.1517) (width 0.254) (layer F.Cu) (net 23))
 (segment (start 185.0809 99.0867) (end 185.0809 99.4042) (width 0.254) (layer F.Cu) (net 23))
 (segment (start 110.30965 111.1517) (end 97.60965 98.4517) (width 0.254) (layer F.Cu) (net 23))
 (segment (start 97.60965 98.4517) (end 97.5627 98.4517) (width 0.254) (layer F.Cu) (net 23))
 (segment (start 99.949 88.392) (end 100.457 88.392) (width 0.254) (layer F.Cu) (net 23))
 (segment (start 97.5627 90.7783) (end 99.949 88.392) (width 0.254) (layer F.Cu) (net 23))
 (segment (start 97.5627 98.6054) (end 97.5627 90.7783) (width 0.254) (layer F.Cu) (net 23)))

